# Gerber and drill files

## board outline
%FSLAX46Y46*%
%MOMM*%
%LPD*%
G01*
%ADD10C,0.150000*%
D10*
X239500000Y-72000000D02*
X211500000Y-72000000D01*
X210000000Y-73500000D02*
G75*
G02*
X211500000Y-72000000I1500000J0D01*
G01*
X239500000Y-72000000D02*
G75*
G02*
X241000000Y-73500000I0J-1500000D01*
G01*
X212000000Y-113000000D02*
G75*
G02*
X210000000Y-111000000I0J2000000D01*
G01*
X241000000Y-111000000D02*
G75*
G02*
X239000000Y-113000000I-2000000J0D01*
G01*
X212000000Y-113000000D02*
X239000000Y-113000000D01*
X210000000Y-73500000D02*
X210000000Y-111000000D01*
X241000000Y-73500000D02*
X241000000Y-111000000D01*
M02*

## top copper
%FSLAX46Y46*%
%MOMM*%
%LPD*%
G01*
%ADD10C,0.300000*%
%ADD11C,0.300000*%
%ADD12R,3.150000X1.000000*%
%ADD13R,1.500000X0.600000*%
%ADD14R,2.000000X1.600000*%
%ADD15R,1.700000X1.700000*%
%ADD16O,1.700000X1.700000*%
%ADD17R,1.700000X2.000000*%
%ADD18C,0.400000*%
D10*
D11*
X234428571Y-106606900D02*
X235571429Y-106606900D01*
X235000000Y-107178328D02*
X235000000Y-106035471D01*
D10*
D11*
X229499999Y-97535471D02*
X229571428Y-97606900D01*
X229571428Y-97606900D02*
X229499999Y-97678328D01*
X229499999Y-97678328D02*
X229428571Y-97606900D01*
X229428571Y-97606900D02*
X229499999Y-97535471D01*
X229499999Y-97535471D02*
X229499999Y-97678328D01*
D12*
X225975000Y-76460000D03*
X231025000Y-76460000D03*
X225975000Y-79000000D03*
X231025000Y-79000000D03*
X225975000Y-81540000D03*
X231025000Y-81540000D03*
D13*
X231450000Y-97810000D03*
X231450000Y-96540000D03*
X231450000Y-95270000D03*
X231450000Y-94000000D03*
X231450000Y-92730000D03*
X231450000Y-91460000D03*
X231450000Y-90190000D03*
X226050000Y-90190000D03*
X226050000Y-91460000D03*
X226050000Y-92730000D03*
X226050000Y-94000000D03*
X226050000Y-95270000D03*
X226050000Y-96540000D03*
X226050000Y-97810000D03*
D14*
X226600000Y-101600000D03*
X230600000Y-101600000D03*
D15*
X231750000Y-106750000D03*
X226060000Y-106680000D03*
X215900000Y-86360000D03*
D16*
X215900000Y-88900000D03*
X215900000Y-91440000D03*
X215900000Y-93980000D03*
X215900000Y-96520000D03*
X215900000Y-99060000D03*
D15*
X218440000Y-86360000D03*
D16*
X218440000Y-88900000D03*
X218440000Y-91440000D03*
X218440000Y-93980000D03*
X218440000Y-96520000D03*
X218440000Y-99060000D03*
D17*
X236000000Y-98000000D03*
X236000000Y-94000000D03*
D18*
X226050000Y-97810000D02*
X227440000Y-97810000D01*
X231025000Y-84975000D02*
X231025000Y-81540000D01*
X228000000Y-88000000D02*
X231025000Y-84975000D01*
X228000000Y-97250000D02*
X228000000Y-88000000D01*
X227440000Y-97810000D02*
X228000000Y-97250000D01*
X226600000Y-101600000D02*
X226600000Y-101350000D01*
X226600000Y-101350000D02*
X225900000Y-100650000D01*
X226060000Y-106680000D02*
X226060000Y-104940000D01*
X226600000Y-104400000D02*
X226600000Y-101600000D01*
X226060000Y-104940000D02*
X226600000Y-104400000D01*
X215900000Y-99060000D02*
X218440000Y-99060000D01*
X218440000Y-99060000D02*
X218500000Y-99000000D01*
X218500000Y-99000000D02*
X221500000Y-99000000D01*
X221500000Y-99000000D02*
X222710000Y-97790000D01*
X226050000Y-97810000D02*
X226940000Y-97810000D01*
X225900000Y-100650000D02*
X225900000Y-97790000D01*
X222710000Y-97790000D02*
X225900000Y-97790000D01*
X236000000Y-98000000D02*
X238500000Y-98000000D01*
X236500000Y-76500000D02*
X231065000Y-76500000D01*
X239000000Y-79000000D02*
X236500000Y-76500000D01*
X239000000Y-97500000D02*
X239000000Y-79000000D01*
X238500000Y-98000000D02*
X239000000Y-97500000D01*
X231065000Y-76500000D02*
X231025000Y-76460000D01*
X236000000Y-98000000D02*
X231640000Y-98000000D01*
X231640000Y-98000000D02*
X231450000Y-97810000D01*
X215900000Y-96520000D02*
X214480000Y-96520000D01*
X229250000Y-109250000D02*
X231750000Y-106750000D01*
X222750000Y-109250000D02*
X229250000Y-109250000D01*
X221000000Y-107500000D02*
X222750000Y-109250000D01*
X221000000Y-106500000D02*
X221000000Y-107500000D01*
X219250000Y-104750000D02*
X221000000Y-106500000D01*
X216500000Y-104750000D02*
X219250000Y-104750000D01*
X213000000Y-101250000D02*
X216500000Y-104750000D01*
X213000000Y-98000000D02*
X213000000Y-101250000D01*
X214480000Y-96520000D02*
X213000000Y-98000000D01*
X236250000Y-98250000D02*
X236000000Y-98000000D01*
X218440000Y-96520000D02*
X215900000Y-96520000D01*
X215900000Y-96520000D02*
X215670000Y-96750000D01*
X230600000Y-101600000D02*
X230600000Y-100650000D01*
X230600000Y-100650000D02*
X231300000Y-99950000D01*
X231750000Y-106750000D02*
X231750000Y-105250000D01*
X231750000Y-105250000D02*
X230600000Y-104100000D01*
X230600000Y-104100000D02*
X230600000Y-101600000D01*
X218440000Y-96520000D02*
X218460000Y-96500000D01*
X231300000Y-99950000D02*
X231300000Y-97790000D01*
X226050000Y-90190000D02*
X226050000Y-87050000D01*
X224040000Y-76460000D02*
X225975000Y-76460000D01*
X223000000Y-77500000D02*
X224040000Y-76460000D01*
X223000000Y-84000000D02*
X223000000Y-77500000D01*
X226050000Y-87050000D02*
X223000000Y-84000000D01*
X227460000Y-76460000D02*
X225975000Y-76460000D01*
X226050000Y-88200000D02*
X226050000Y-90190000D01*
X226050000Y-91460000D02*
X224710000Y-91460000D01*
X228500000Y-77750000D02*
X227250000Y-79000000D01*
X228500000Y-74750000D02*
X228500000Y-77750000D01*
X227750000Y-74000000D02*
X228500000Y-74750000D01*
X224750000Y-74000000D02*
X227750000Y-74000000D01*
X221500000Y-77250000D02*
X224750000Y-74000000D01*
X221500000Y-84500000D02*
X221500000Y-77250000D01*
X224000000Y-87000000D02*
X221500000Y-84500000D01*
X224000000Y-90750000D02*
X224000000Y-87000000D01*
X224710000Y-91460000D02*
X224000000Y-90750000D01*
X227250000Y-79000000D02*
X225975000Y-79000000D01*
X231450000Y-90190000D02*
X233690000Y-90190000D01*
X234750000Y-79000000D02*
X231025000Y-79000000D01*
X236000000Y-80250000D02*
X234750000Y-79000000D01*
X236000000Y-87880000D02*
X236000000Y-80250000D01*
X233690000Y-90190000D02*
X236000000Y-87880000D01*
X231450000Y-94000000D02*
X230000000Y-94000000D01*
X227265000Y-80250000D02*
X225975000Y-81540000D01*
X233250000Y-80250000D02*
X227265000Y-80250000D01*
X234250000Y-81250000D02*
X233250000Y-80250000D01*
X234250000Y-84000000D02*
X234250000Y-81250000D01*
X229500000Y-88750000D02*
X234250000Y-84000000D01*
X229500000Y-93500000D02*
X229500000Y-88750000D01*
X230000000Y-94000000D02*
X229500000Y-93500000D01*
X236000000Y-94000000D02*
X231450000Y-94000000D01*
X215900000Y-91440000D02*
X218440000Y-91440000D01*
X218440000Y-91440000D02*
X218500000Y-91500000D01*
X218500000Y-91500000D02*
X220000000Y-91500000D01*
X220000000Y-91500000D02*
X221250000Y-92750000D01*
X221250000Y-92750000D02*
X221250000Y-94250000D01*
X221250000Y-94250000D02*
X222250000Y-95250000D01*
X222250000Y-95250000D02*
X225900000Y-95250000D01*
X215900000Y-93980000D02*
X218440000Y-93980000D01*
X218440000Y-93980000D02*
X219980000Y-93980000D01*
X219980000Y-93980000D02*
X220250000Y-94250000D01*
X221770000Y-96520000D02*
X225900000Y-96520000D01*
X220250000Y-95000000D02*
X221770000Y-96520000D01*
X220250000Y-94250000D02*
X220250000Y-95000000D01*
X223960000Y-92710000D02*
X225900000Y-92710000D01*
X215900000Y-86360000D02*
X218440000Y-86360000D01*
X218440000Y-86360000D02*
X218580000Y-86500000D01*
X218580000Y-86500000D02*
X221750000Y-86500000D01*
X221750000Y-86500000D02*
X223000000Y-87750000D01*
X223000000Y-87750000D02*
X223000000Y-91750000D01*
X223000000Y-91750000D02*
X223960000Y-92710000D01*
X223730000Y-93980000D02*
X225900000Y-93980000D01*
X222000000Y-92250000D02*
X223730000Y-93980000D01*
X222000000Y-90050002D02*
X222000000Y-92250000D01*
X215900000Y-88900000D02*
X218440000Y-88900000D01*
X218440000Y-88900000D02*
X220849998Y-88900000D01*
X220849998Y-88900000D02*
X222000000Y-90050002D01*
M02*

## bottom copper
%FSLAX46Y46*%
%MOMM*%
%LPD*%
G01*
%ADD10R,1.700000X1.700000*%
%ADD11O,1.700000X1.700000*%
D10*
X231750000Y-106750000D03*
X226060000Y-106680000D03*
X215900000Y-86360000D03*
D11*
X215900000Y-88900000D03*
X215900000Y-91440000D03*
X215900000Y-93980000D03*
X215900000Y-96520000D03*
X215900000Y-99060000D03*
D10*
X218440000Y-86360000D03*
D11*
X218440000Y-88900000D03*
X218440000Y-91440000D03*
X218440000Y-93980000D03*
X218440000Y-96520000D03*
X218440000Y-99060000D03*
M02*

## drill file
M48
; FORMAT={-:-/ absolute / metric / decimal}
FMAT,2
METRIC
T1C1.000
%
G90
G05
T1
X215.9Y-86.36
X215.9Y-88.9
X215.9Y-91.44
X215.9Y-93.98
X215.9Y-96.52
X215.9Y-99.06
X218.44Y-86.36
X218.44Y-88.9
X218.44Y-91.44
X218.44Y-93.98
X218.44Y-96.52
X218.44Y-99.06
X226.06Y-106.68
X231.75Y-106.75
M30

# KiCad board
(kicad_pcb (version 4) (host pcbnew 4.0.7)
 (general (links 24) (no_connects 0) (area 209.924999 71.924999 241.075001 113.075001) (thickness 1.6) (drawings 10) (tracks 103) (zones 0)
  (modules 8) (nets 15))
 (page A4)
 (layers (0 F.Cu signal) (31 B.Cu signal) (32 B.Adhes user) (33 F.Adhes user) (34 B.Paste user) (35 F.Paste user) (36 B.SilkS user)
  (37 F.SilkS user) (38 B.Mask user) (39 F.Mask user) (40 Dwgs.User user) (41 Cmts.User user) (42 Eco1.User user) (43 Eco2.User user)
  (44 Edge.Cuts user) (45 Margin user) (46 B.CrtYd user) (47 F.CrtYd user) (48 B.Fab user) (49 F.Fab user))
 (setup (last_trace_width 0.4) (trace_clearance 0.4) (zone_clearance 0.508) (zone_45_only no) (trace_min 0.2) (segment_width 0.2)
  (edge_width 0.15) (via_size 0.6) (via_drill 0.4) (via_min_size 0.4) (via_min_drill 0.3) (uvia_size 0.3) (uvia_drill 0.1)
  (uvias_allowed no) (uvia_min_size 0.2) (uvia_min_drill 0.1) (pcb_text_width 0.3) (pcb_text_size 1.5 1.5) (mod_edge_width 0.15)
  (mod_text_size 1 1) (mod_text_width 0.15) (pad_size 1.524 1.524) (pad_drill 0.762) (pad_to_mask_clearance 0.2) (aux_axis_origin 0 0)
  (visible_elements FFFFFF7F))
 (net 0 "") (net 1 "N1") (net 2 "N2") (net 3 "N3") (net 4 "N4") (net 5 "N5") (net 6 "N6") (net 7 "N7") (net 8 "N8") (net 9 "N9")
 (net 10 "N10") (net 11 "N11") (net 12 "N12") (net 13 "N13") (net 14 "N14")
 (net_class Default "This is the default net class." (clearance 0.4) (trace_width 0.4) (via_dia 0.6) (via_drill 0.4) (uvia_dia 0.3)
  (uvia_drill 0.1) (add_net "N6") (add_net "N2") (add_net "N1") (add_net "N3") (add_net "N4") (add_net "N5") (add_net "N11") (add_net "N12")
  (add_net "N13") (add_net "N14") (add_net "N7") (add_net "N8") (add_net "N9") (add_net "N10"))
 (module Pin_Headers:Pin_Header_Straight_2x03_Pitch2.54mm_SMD (layer F.Cu) (at 228.5 79)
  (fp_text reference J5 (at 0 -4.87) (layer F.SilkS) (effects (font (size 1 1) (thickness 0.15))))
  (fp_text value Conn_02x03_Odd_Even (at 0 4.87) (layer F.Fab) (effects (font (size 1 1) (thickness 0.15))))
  (pad 1 smd rect (at -2.525 -2.54) (size 3.15 1) (layers F.Cu F.Paste F.Mask) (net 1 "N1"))
  (pad 2 smd rect (at 2.525 -2.54) (size 3.15 1) (layers F.Cu F.Paste F.Mask) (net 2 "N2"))
  (pad 3 smd rect (at -2.525 0) (size 3.15 1) (layers F.Cu F.Paste F.Mask) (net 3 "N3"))
  (pad 4 smd rect (at 2.525 0) (size 3.15 1) (layers F.Cu F.Paste F.Mask) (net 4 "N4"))
  (pad 5 smd rect (at -2.525 2.54) (size 3.15 1) (layers F.Cu F.Paste F.Mask) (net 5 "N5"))
  (pad 6 smd rect (at 2.525 2.54) (size 3.15 1) (layers F.Cu F.Paste F.Mask) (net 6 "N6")))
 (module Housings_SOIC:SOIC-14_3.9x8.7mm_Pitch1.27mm (layer F.Cu) (at 228.75 94 180)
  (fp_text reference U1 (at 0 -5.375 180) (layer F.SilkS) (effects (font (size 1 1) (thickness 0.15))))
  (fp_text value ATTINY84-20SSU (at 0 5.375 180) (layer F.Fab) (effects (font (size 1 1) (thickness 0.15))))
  (pad 1 smd rect (at -2.7 -3.81 180) (size 1.5 0.6) (layers F.Cu F.Paste F.Mask) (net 2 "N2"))
  (pad 2 smd rect (at -2.7 -2.54 180) (size 1.5 0.6) (layers F.Cu F.Paste F.Mask) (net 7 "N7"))
  (pad 3 smd rect (at -2.7 -1.27 180) (size 1.5 0.6) (layers F.Cu F.Paste F.Mask) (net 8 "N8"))
  (pad 4 smd rect (at -2.7 0 180) (size 1.5 0.6) (layers F.Cu F.Paste F.Mask) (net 5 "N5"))
  (pad 5 smd rect (at -2.7 1.27 180) (size 1.5 0.6) (layers F.Cu F.Paste F.Mask) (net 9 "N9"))
  (pad 6 smd rect (at -2.7 2.54 180) (size 1.5 0.6) (layers F.Cu F.Paste F.Mask) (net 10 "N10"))
  (pad 7 smd rect (at -2.7 3.81 180) (size 1.5 0.6) (layers F.Cu F.Paste F.Mask) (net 4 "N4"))
  (pad 8 smd rect (at 2.7 3.81 180) (size 1.5 0.6) (layers F.Cu F.Paste F.Mask) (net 1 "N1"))
  (pad 9 smd rect (at 2.7 2.54 180) (size 1.5 0.6) (layers F.Cu F.Paste F.Mask) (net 3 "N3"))
  (pad 10 smd rect (at 2.7 1.27 180) (size 1.5 0.6) (layers F.Cu F.Paste F.Mask) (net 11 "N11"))
  (pad 11 smd rect (at 2.7 0 180) (size 1.5 0.6) (layers F.Cu F.Paste F.Mask) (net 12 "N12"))
  (pad 12 smd rect (at 2.7 -1.27 180) (size 1.5 0.6) (layers F.Cu F.Paste F.Mask) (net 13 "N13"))
  (pad 13 smd rect (at 2.7 -2.54 180) (size 1.5 0.6) (layers F.Cu F.Paste F.Mask) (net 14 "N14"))
  (pad 14 smd rect (at 2.7 -3.81 180) (size 1.5 0.6) (layers F.Cu F.Paste F.Mask) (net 6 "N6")))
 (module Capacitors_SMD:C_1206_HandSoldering (layer F.Cu) (at 228.6 101.6)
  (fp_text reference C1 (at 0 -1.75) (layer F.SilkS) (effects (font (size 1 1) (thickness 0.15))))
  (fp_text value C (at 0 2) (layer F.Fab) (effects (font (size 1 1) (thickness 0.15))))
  (pad 1 smd rect (at -2 0) (size 2 1.6) (layers F.Cu F.Paste F.Mask) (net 6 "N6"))
  (pad 2 smd rect (at 2 0) (size 2 1.6) (layers F.Cu F.Paste F.Mask) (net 2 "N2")))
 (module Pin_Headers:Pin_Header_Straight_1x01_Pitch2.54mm (layer F.Cu) (at 231.75 106.75)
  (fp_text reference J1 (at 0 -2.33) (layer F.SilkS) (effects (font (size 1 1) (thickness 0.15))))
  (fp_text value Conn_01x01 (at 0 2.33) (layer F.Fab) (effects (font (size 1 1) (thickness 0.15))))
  (pad 1 thru_hole rect (at 0 0) (size 1.7 1.7) (drill 1) (layers *.Cu *.Mask) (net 2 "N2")))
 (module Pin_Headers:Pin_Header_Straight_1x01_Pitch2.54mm (layer F.Cu) (at 226.06 106.68)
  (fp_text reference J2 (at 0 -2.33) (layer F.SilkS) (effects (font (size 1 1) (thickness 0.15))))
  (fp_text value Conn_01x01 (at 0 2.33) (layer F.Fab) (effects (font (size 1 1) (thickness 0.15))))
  (pad 1 thru_hole rect (at 0 0) (size 1.7 1.7) (drill 1) (layers *.Cu *.Mask) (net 6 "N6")))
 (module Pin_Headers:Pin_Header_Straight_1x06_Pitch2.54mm (layer F.Cu) (at 215.9 86.36)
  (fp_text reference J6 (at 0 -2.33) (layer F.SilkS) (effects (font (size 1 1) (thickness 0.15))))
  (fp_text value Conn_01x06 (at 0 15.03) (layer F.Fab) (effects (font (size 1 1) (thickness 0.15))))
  (pad 1 thru_hole rect (at 0 0) (size 1.7 1.7) (drill 1) (layers *.Cu *.Mask) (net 11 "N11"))
  (pad 2 thru_hole oval (at 0 2.54) (size 1.7 1.7) (drill 1) (layers *.Cu *.Mask) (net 12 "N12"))
  (pad 3 thru_hole oval (at 0 5.08) (size 1.7 1.7) (drill 1) (layers *.Cu *.Mask) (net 13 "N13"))
  (pad 4 thru_hole oval (at 0 7.62) (size 1.7 1.7) (drill 1) (layers *.Cu *.Mask) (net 14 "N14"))
  (pad 5 thru_hole oval (at 0 10.16) (size 1.7 1.7) (drill 1) (layers *.Cu *.Mask) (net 2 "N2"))
  (pad 6 thru_hole oval (at 0 12.7) (size 1.7 1.7) (drill 1) (layers *.Cu *.Mask) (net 6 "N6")))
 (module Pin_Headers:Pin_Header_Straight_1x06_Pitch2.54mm (layer F.Cu) (at 218.44 86.36)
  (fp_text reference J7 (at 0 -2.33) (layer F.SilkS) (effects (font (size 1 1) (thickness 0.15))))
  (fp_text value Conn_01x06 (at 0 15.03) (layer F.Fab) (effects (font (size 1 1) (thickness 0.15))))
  (pad 1 thru_hole rect (at 0 0) (size 1.7 1.7) (drill 1) (layers *.Cu *.Mask) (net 11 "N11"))
  (pad 2 thru_hole oval (at 0 2.54) (size 1.7 1.7) (drill 1) (layers *.Cu *.Mask) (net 12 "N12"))
  (pad 3 thru_hole oval (at 0 5.08) (size 1.7 1.7) (drill 1) (layers *.Cu *.Mask) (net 13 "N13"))
  (pad 4 thru_hole oval (at 0 7.62) (size 1.7 1.7) (drill 1) (layers *.Cu *.Mask) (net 14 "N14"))
  (pad 5 thru_hole oval (at 0 10.16) (size 1.7 1.7) (drill 1) (layers *.Cu *.Mask) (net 2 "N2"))
  (pad 6 thru_hole oval (at 0 12.7) (size 1.7 1.7) (drill 1) (layers *.Cu *.Mask) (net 6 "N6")))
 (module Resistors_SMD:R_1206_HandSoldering (layer F.Cu) (at 236 96 90)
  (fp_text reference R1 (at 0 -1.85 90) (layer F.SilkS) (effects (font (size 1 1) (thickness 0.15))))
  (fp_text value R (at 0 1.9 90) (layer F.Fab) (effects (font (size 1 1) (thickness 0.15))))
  (pad 1 smd rect (at -2 0 90) (size 2 1.7) (layers F.Cu F.Paste F.Mask) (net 2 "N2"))
  (pad 2 smd rect (at 2 0 90) (size 2 1.7) (layers F.Cu F.Paste F.Mask) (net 5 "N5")))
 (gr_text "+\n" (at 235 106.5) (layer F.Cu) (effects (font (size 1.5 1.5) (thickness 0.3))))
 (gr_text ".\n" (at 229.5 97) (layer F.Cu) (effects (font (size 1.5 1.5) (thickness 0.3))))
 (gr_line (start 239.5 72) (end 211.5 72) (angle 90) (layer Edge.Cuts) (width 0.15))
 (gr_arc (start 211.5 73.5) (end 210 73.5) (angle 90) (layer Edge.Cuts) (width 0.15))
 (gr_arc (start 239.5 73.5) (end 239.5 72) (angle 90) (layer Edge.Cuts) (width 0.15))
 (gr_arc (start 212 111) (end 212 113) (angle 90) (layer Edge.Cuts) (width 0.15))
 (gr_arc (start 239 111) (end 241 111) (angle 90) (layer Edge.Cuts) (width 0.15))
 (gr_line (start 212 113) (end 239 113) (angle 90) (layer Edge.Cuts) (width 0.15))
 (gr_line (start 210 73.5) (end 210 111) (angle 90) (layer Edge.Cuts) (width 0.15))
 (gr_line (start 241 73.5) (end 241 111) (angle 90) (layer Edge.Cuts) (width 0.15))
 (segment (start 226.05 97.81) (end 227.44 97.81) (width 0.4) (layer F.Cu) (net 6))
 (segment (start 231.025 84.975) (end 231.025 81.54) (width 0.4) (layer F.Cu) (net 6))
 (segment (start 228 88) (end 231.025 84.975) (width 0.4) (layer F.Cu) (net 6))
 (segment (start 228 97.25) (end 228 88) (width 0.4) (layer F.Cu) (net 6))
 (segment (start 227.44 97.81) (end 228 97.25) (width 0.4) (layer F.Cu) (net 6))
 (segment (start 226.6 101.6) (end 226.6 101.35) (width 0.4) (layer F.Cu) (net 6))
 (segment (start 226.6 101.35) (end 225.9 100.65) (width 0.4) (layer F.Cu) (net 6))
 (segment (start 226.06 106.68) (end 226.06 104.94) (width 0.4) (layer F.Cu) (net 6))
 (segment (start 226.6 104.4) (end 226.6 101.6) (width 0.4) (layer F.Cu) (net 6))
 (segment (start 226.06 104.94) (end 226.6 104.4) (width 0.4) (layer F.Cu) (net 6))
 (segment (start 215.9 99.06) (end 218.44 99.06) (width 0.4) (layer F.Cu) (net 6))
 (segment (start 218.44 99.06) (end 218.5 99) (width 0.4) (layer F.Cu) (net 6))
 (segment (start 218.5 99) (end 221.5 99) (width 0.4) (layer F.Cu) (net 6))
 (segment (start 221.5 99) (end 222.71 97.79) (width 0.4) (layer F.Cu) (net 6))
 (segment (start 226.05 97.81) (end 226.94 97.81) (width 0.4) (layer F.Cu) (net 6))
 (segment (start 225.9 100.65) (end 225.9 97.79) (width 0.4) (layer F.Cu) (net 6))
 (segment (start 222.71 97.79) (end 225.9 97.79) (width 0.4) (layer F.Cu) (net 6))
 (segment (start 236 98) (end 238.5 98) (width 0.4) (layer F.Cu) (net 2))
 (segment (start 236.5 76.5) (end 231.065 76.5) (width 0.4) (layer F.Cu) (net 2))
 (segment (start 239 79) (end 236.5 76.5) (width 0.4) (layer F.Cu) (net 2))
 (segment (start 239 97.5) (end 239 79) (width 0.4) (layer F.Cu) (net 2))
 (segment (start 238.5 98) (end 239 97.5) (width 0.4) (layer F.Cu) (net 2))
 (segment (start 231.065 76.5) (end 231.025 76.46) (width 0.4) (layer F.Cu) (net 2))
 (segment (start 236 98) (end 231.64 98) (width 0.4) (layer F.Cu) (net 2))
 (segment (start 231.64 98) (end 231.45 97.81) (width 0.4) (layer F.Cu) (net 2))
 (segment (start 215.9 96.52) (end 214.48 96.52) (width 0.4) (layer F.Cu) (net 2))
 (segment (start 229.25 109.25) (end 231.75 106.75) (width 0.4) (layer F.Cu) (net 2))
 (segment (start 222.75 109.25) (end 229.25 109.25) (width 0.4) (layer F.Cu) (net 2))
 (segment (start 221 107.5) (end 222.75 109.25) (width 0.4) (layer F.Cu) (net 2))
 (segment (start 221 106.5) (end 221 107.5) (width 0.4) (layer F.Cu) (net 2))
 (segment (start 219.25 104.75) (end 221 106.5) (width 0.4) (layer F.Cu) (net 2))
 (segment (start 216.5 104.75) (end 219.25 104.75) (width 0.4) (layer F.Cu) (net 2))
 (segment (start 213 101.25) (end 216.5 104.75) (width 0.4) (layer F.Cu) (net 2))
 (segment (start 213 98) (end 213 101.25) (width 0.4) (layer F.Cu) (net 2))
 (segment (start 214.48 96.52) (end 213 98) (width 0.4) (layer F.Cu) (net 2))
 (segment (start 236.25 98.25) (end 236 98) (width 0.4) (layer F.Cu) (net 2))
 (segment (start 218.44 96.52) (end 215.9 96.52) (width 0.4) (layer F.Cu) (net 2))
 (segment (start 215.9 96.52) (end 215.67 96.75) (width 0.4) (layer F.Cu) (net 2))
 (segment (start 230.6 101.6) (end 230.6 100.65) (width 0.4) (layer F.Cu) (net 2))
 (segment (start 230.6 100.65) (end 231.3 99.95) (width 0.4) (layer F.Cu) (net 2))
 (segment (start 231.75 106.75) (end 231.75 105.25) (width 0.4) (layer F.Cu) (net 2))
 (segment (start 231.75 105.25) (end 230.6 104.1) (width 0.4) (layer F.Cu) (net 2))
 (segment (start 230.6 104.1) (end 230.6 101.6) (width 0.4) (layer F.Cu) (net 2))
 (segment (start 218.44 96.52) (end 218.46 96.5) (width 0.4) (layer F.Cu) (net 2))
 (segment (start 231.3 99.95) (end 231.3 97.79) (width 0.4) (layer F.Cu) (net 2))
 (segment (start 226.05 90.19) (end 226.05 87.05) (width 0.4) (layer F.Cu) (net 1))
 (segment (start 224.04 76.46) (end 225.975 76.46) (width 0.4) (layer F.Cu) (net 1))
 (segment (start 223 77.5) (end 224.04 76.46) (width 0.4) (layer F.Cu) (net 1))
 (segment (start 223 84) (end 223 77.5) (width 0.4) (layer F.Cu) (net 1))
 (segment (start 226.05 87.05) (end 223 84) (width 0.4) (layer F.Cu) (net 1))
 (segment (start 227.46 76.46) (end 225.975 76.46) (width 0.4) (layer F.Cu) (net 1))
 (segment (start 226.05 88.2) (end 226.05 90.19) (width 0.4) (layer F.Cu) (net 1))
 (segment (start 226.05 91.46) (end 224.71 91.46) (width 0.4) (layer F.Cu) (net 3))
 (segment (start 228.5 77.75) (end 227.25 79) (width 0.4) (layer F.Cu) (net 3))
 (segment (start 228.5 74.75) (end 228.5 77.75) (width 0.4) (layer F.Cu) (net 3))
 (segment (start 227.75 74) (end 228.5 74.75) (width 0.4) (layer F.Cu) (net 3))
 (segment (start 224.75 74) (end 227.75 74) (width 0.4) (layer F.Cu) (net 3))
 (segment (start 221.5 77.25) (end 224.75 74) (width 0.4) (layer F.Cu) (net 3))
 (segment (start 221.5 84.5) (end 221.5 77.25) (width 0.4) (layer F.Cu) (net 3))
 (segment (start 224 87) (end 221.5 84.5) (width 0.4) (layer F.Cu) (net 3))
 (segment (start 224 90.75) (end 224 87) (width 0.4) (layer F.Cu) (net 3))
 (segment (start 224.71 91.46) (end 224 90.75) (width 0.4) (layer F.Cu) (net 3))
 (segment (start 227.25 79) (end 225.975 79) (width 0.4) (layer F.Cu) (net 3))
 (segment (start 231.45 90.19) (end 233.69 90.19) (width 0.4) (layer F.Cu) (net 4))
 (segment (start 234.75 79) (end 231.025 79) (width 0.4) (layer F.Cu) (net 4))
 (segment (start 236 80.25) (end 234.75 79) (width 0.4) (layer F.Cu) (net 4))
 (segment (start 236 87.88) (end 236 80.25) (width 0.4) (layer F.Cu) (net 4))
 (segment (start 233.69 90.19) (end 236 87.88) (width 0.4) (layer F.Cu) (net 4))
 (segment (start 231.45 94) (end 230 94) (width 0.4) (layer F.Cu) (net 5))
 (segment (start 227.265 80.25) (end 225.975 81.54) (width 0.4) (layer F.Cu) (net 5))
 (segment (start 233.25 80.25) (end 227.265 80.25) (width 0.4) (layer F.Cu) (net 5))
 (segment (start 234.25 81.25) (end 233.25 80.25) (width 0.4) (layer F.Cu) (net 5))
 (segment (start 234.25 84) (end 234.25 81.25) (width 0.4) (layer F.Cu) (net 5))
 (segment (start 229.5 88.75) (end 234.25 84) (width 0.4) (layer F.Cu) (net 5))
 (segment (start 229.5 93.5) (end 229.5 88.75) (width 0.4) (layer F.Cu) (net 5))
 (segment (start 230 94) (end 229.5 93.5) (width 0.4) (layer F.Cu) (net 5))
 (segment (start 236 94) (end 231.45 94) (width 0.4) (layer F.Cu) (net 5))
 (segment (start 215.9 91.44) (end 218.44 91.44) (width 0.4) (layer F.Cu) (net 13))
 (segment (start 218.44 91.44) (end 218.5 91.5) (width 0.4) (layer F.Cu) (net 13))
 (segment (start 218.5 91.5) (end 220 91.5) (width 0.4) (layer F.Cu) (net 13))
 (segment (start 220 91.5) (end 221.25 92.75) (width 0.4) (layer F.Cu) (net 13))
 (segment (start 221.25 92.75) (end 221.25 94.25) (width 0.4) (layer F.Cu) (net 13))
 (segment (start 221.25 94.25) (end 222.25 95.25) (width 0.4) (layer F.Cu) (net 13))
 (segment (start 222.25 95.25) (end 225.9 95.25) (width 0.4) (layer F.Cu) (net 13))
 (segment (start 215.9 93.98) (end 218.44 93.98) (width 0.4) (layer F.Cu) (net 14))
 (segment (start 218.44 93.98) (end 219.98 93.98) (width 0.4) (layer F.Cu) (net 14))
 (segment (start 219.98 93.98) (end 220.25 94.25) (width 0.4) (layer F.Cu) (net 14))
 (segment (start 221.77 96.52) (end 225.9 96.52) (width 0.4) (layer F.Cu) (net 14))
 (segment (start 220.25 95) (end 221.77 96.52) (width 0.4) (layer F.Cu) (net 14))
 (segment (start 220.25 94.25) (end 220.25 95) (width 0.4) (layer F.Cu) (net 14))
 (segment (start 223.96 92.71) (end 225.9 92.71) (width 0.4) (layer F.Cu) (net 11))
 (segment (start 215.9 86.36) (end 218.44 86.36) (width 0.4) (layer F.Cu) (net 11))
 (segment (start 218.44 86.36) (end 218.58 86.5) (width 0.4) (layer F.Cu) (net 11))
 (segment (start 218.58 86.5) (end 221.75 86.5) (width 0.4) (layer F.Cu) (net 11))
 (segment (start 221.75 86.5) (end 223 87.75) (width 0.4) (layer F.Cu) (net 11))
 (segment (start 223 87.75) (end 223 91.75) (width 0.4) (layer F.Cu) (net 11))
 (segment (start 223 91.75) (end 223.96 92.71) (width 0.4) (layer F.Cu) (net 11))
 (segment (start 223.73 93.98) (end 225.9 93.98) (width 0.4) (layer F.Cu) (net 12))
 (segment (start 222 92.25) (end 223.73 93.98) (width 0.4) (layer F.Cu) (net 12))
 (segment (start 222 90.050002) (end 222 92.25) (width 0.4) (layer F.Cu) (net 12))
 (segment (start 215.9 88.9) (end 218.44 88.9) (width 0.4) (layer F.Cu) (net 12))
 (segment (start 218.44 88.9) (end 220.849998 88.9) (width 0.4) (layer F.Cu) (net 12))
 (segment (start 220.849998 88.9) (end 222 90.050002) (width 0.4) (layer F.Cu) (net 12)))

